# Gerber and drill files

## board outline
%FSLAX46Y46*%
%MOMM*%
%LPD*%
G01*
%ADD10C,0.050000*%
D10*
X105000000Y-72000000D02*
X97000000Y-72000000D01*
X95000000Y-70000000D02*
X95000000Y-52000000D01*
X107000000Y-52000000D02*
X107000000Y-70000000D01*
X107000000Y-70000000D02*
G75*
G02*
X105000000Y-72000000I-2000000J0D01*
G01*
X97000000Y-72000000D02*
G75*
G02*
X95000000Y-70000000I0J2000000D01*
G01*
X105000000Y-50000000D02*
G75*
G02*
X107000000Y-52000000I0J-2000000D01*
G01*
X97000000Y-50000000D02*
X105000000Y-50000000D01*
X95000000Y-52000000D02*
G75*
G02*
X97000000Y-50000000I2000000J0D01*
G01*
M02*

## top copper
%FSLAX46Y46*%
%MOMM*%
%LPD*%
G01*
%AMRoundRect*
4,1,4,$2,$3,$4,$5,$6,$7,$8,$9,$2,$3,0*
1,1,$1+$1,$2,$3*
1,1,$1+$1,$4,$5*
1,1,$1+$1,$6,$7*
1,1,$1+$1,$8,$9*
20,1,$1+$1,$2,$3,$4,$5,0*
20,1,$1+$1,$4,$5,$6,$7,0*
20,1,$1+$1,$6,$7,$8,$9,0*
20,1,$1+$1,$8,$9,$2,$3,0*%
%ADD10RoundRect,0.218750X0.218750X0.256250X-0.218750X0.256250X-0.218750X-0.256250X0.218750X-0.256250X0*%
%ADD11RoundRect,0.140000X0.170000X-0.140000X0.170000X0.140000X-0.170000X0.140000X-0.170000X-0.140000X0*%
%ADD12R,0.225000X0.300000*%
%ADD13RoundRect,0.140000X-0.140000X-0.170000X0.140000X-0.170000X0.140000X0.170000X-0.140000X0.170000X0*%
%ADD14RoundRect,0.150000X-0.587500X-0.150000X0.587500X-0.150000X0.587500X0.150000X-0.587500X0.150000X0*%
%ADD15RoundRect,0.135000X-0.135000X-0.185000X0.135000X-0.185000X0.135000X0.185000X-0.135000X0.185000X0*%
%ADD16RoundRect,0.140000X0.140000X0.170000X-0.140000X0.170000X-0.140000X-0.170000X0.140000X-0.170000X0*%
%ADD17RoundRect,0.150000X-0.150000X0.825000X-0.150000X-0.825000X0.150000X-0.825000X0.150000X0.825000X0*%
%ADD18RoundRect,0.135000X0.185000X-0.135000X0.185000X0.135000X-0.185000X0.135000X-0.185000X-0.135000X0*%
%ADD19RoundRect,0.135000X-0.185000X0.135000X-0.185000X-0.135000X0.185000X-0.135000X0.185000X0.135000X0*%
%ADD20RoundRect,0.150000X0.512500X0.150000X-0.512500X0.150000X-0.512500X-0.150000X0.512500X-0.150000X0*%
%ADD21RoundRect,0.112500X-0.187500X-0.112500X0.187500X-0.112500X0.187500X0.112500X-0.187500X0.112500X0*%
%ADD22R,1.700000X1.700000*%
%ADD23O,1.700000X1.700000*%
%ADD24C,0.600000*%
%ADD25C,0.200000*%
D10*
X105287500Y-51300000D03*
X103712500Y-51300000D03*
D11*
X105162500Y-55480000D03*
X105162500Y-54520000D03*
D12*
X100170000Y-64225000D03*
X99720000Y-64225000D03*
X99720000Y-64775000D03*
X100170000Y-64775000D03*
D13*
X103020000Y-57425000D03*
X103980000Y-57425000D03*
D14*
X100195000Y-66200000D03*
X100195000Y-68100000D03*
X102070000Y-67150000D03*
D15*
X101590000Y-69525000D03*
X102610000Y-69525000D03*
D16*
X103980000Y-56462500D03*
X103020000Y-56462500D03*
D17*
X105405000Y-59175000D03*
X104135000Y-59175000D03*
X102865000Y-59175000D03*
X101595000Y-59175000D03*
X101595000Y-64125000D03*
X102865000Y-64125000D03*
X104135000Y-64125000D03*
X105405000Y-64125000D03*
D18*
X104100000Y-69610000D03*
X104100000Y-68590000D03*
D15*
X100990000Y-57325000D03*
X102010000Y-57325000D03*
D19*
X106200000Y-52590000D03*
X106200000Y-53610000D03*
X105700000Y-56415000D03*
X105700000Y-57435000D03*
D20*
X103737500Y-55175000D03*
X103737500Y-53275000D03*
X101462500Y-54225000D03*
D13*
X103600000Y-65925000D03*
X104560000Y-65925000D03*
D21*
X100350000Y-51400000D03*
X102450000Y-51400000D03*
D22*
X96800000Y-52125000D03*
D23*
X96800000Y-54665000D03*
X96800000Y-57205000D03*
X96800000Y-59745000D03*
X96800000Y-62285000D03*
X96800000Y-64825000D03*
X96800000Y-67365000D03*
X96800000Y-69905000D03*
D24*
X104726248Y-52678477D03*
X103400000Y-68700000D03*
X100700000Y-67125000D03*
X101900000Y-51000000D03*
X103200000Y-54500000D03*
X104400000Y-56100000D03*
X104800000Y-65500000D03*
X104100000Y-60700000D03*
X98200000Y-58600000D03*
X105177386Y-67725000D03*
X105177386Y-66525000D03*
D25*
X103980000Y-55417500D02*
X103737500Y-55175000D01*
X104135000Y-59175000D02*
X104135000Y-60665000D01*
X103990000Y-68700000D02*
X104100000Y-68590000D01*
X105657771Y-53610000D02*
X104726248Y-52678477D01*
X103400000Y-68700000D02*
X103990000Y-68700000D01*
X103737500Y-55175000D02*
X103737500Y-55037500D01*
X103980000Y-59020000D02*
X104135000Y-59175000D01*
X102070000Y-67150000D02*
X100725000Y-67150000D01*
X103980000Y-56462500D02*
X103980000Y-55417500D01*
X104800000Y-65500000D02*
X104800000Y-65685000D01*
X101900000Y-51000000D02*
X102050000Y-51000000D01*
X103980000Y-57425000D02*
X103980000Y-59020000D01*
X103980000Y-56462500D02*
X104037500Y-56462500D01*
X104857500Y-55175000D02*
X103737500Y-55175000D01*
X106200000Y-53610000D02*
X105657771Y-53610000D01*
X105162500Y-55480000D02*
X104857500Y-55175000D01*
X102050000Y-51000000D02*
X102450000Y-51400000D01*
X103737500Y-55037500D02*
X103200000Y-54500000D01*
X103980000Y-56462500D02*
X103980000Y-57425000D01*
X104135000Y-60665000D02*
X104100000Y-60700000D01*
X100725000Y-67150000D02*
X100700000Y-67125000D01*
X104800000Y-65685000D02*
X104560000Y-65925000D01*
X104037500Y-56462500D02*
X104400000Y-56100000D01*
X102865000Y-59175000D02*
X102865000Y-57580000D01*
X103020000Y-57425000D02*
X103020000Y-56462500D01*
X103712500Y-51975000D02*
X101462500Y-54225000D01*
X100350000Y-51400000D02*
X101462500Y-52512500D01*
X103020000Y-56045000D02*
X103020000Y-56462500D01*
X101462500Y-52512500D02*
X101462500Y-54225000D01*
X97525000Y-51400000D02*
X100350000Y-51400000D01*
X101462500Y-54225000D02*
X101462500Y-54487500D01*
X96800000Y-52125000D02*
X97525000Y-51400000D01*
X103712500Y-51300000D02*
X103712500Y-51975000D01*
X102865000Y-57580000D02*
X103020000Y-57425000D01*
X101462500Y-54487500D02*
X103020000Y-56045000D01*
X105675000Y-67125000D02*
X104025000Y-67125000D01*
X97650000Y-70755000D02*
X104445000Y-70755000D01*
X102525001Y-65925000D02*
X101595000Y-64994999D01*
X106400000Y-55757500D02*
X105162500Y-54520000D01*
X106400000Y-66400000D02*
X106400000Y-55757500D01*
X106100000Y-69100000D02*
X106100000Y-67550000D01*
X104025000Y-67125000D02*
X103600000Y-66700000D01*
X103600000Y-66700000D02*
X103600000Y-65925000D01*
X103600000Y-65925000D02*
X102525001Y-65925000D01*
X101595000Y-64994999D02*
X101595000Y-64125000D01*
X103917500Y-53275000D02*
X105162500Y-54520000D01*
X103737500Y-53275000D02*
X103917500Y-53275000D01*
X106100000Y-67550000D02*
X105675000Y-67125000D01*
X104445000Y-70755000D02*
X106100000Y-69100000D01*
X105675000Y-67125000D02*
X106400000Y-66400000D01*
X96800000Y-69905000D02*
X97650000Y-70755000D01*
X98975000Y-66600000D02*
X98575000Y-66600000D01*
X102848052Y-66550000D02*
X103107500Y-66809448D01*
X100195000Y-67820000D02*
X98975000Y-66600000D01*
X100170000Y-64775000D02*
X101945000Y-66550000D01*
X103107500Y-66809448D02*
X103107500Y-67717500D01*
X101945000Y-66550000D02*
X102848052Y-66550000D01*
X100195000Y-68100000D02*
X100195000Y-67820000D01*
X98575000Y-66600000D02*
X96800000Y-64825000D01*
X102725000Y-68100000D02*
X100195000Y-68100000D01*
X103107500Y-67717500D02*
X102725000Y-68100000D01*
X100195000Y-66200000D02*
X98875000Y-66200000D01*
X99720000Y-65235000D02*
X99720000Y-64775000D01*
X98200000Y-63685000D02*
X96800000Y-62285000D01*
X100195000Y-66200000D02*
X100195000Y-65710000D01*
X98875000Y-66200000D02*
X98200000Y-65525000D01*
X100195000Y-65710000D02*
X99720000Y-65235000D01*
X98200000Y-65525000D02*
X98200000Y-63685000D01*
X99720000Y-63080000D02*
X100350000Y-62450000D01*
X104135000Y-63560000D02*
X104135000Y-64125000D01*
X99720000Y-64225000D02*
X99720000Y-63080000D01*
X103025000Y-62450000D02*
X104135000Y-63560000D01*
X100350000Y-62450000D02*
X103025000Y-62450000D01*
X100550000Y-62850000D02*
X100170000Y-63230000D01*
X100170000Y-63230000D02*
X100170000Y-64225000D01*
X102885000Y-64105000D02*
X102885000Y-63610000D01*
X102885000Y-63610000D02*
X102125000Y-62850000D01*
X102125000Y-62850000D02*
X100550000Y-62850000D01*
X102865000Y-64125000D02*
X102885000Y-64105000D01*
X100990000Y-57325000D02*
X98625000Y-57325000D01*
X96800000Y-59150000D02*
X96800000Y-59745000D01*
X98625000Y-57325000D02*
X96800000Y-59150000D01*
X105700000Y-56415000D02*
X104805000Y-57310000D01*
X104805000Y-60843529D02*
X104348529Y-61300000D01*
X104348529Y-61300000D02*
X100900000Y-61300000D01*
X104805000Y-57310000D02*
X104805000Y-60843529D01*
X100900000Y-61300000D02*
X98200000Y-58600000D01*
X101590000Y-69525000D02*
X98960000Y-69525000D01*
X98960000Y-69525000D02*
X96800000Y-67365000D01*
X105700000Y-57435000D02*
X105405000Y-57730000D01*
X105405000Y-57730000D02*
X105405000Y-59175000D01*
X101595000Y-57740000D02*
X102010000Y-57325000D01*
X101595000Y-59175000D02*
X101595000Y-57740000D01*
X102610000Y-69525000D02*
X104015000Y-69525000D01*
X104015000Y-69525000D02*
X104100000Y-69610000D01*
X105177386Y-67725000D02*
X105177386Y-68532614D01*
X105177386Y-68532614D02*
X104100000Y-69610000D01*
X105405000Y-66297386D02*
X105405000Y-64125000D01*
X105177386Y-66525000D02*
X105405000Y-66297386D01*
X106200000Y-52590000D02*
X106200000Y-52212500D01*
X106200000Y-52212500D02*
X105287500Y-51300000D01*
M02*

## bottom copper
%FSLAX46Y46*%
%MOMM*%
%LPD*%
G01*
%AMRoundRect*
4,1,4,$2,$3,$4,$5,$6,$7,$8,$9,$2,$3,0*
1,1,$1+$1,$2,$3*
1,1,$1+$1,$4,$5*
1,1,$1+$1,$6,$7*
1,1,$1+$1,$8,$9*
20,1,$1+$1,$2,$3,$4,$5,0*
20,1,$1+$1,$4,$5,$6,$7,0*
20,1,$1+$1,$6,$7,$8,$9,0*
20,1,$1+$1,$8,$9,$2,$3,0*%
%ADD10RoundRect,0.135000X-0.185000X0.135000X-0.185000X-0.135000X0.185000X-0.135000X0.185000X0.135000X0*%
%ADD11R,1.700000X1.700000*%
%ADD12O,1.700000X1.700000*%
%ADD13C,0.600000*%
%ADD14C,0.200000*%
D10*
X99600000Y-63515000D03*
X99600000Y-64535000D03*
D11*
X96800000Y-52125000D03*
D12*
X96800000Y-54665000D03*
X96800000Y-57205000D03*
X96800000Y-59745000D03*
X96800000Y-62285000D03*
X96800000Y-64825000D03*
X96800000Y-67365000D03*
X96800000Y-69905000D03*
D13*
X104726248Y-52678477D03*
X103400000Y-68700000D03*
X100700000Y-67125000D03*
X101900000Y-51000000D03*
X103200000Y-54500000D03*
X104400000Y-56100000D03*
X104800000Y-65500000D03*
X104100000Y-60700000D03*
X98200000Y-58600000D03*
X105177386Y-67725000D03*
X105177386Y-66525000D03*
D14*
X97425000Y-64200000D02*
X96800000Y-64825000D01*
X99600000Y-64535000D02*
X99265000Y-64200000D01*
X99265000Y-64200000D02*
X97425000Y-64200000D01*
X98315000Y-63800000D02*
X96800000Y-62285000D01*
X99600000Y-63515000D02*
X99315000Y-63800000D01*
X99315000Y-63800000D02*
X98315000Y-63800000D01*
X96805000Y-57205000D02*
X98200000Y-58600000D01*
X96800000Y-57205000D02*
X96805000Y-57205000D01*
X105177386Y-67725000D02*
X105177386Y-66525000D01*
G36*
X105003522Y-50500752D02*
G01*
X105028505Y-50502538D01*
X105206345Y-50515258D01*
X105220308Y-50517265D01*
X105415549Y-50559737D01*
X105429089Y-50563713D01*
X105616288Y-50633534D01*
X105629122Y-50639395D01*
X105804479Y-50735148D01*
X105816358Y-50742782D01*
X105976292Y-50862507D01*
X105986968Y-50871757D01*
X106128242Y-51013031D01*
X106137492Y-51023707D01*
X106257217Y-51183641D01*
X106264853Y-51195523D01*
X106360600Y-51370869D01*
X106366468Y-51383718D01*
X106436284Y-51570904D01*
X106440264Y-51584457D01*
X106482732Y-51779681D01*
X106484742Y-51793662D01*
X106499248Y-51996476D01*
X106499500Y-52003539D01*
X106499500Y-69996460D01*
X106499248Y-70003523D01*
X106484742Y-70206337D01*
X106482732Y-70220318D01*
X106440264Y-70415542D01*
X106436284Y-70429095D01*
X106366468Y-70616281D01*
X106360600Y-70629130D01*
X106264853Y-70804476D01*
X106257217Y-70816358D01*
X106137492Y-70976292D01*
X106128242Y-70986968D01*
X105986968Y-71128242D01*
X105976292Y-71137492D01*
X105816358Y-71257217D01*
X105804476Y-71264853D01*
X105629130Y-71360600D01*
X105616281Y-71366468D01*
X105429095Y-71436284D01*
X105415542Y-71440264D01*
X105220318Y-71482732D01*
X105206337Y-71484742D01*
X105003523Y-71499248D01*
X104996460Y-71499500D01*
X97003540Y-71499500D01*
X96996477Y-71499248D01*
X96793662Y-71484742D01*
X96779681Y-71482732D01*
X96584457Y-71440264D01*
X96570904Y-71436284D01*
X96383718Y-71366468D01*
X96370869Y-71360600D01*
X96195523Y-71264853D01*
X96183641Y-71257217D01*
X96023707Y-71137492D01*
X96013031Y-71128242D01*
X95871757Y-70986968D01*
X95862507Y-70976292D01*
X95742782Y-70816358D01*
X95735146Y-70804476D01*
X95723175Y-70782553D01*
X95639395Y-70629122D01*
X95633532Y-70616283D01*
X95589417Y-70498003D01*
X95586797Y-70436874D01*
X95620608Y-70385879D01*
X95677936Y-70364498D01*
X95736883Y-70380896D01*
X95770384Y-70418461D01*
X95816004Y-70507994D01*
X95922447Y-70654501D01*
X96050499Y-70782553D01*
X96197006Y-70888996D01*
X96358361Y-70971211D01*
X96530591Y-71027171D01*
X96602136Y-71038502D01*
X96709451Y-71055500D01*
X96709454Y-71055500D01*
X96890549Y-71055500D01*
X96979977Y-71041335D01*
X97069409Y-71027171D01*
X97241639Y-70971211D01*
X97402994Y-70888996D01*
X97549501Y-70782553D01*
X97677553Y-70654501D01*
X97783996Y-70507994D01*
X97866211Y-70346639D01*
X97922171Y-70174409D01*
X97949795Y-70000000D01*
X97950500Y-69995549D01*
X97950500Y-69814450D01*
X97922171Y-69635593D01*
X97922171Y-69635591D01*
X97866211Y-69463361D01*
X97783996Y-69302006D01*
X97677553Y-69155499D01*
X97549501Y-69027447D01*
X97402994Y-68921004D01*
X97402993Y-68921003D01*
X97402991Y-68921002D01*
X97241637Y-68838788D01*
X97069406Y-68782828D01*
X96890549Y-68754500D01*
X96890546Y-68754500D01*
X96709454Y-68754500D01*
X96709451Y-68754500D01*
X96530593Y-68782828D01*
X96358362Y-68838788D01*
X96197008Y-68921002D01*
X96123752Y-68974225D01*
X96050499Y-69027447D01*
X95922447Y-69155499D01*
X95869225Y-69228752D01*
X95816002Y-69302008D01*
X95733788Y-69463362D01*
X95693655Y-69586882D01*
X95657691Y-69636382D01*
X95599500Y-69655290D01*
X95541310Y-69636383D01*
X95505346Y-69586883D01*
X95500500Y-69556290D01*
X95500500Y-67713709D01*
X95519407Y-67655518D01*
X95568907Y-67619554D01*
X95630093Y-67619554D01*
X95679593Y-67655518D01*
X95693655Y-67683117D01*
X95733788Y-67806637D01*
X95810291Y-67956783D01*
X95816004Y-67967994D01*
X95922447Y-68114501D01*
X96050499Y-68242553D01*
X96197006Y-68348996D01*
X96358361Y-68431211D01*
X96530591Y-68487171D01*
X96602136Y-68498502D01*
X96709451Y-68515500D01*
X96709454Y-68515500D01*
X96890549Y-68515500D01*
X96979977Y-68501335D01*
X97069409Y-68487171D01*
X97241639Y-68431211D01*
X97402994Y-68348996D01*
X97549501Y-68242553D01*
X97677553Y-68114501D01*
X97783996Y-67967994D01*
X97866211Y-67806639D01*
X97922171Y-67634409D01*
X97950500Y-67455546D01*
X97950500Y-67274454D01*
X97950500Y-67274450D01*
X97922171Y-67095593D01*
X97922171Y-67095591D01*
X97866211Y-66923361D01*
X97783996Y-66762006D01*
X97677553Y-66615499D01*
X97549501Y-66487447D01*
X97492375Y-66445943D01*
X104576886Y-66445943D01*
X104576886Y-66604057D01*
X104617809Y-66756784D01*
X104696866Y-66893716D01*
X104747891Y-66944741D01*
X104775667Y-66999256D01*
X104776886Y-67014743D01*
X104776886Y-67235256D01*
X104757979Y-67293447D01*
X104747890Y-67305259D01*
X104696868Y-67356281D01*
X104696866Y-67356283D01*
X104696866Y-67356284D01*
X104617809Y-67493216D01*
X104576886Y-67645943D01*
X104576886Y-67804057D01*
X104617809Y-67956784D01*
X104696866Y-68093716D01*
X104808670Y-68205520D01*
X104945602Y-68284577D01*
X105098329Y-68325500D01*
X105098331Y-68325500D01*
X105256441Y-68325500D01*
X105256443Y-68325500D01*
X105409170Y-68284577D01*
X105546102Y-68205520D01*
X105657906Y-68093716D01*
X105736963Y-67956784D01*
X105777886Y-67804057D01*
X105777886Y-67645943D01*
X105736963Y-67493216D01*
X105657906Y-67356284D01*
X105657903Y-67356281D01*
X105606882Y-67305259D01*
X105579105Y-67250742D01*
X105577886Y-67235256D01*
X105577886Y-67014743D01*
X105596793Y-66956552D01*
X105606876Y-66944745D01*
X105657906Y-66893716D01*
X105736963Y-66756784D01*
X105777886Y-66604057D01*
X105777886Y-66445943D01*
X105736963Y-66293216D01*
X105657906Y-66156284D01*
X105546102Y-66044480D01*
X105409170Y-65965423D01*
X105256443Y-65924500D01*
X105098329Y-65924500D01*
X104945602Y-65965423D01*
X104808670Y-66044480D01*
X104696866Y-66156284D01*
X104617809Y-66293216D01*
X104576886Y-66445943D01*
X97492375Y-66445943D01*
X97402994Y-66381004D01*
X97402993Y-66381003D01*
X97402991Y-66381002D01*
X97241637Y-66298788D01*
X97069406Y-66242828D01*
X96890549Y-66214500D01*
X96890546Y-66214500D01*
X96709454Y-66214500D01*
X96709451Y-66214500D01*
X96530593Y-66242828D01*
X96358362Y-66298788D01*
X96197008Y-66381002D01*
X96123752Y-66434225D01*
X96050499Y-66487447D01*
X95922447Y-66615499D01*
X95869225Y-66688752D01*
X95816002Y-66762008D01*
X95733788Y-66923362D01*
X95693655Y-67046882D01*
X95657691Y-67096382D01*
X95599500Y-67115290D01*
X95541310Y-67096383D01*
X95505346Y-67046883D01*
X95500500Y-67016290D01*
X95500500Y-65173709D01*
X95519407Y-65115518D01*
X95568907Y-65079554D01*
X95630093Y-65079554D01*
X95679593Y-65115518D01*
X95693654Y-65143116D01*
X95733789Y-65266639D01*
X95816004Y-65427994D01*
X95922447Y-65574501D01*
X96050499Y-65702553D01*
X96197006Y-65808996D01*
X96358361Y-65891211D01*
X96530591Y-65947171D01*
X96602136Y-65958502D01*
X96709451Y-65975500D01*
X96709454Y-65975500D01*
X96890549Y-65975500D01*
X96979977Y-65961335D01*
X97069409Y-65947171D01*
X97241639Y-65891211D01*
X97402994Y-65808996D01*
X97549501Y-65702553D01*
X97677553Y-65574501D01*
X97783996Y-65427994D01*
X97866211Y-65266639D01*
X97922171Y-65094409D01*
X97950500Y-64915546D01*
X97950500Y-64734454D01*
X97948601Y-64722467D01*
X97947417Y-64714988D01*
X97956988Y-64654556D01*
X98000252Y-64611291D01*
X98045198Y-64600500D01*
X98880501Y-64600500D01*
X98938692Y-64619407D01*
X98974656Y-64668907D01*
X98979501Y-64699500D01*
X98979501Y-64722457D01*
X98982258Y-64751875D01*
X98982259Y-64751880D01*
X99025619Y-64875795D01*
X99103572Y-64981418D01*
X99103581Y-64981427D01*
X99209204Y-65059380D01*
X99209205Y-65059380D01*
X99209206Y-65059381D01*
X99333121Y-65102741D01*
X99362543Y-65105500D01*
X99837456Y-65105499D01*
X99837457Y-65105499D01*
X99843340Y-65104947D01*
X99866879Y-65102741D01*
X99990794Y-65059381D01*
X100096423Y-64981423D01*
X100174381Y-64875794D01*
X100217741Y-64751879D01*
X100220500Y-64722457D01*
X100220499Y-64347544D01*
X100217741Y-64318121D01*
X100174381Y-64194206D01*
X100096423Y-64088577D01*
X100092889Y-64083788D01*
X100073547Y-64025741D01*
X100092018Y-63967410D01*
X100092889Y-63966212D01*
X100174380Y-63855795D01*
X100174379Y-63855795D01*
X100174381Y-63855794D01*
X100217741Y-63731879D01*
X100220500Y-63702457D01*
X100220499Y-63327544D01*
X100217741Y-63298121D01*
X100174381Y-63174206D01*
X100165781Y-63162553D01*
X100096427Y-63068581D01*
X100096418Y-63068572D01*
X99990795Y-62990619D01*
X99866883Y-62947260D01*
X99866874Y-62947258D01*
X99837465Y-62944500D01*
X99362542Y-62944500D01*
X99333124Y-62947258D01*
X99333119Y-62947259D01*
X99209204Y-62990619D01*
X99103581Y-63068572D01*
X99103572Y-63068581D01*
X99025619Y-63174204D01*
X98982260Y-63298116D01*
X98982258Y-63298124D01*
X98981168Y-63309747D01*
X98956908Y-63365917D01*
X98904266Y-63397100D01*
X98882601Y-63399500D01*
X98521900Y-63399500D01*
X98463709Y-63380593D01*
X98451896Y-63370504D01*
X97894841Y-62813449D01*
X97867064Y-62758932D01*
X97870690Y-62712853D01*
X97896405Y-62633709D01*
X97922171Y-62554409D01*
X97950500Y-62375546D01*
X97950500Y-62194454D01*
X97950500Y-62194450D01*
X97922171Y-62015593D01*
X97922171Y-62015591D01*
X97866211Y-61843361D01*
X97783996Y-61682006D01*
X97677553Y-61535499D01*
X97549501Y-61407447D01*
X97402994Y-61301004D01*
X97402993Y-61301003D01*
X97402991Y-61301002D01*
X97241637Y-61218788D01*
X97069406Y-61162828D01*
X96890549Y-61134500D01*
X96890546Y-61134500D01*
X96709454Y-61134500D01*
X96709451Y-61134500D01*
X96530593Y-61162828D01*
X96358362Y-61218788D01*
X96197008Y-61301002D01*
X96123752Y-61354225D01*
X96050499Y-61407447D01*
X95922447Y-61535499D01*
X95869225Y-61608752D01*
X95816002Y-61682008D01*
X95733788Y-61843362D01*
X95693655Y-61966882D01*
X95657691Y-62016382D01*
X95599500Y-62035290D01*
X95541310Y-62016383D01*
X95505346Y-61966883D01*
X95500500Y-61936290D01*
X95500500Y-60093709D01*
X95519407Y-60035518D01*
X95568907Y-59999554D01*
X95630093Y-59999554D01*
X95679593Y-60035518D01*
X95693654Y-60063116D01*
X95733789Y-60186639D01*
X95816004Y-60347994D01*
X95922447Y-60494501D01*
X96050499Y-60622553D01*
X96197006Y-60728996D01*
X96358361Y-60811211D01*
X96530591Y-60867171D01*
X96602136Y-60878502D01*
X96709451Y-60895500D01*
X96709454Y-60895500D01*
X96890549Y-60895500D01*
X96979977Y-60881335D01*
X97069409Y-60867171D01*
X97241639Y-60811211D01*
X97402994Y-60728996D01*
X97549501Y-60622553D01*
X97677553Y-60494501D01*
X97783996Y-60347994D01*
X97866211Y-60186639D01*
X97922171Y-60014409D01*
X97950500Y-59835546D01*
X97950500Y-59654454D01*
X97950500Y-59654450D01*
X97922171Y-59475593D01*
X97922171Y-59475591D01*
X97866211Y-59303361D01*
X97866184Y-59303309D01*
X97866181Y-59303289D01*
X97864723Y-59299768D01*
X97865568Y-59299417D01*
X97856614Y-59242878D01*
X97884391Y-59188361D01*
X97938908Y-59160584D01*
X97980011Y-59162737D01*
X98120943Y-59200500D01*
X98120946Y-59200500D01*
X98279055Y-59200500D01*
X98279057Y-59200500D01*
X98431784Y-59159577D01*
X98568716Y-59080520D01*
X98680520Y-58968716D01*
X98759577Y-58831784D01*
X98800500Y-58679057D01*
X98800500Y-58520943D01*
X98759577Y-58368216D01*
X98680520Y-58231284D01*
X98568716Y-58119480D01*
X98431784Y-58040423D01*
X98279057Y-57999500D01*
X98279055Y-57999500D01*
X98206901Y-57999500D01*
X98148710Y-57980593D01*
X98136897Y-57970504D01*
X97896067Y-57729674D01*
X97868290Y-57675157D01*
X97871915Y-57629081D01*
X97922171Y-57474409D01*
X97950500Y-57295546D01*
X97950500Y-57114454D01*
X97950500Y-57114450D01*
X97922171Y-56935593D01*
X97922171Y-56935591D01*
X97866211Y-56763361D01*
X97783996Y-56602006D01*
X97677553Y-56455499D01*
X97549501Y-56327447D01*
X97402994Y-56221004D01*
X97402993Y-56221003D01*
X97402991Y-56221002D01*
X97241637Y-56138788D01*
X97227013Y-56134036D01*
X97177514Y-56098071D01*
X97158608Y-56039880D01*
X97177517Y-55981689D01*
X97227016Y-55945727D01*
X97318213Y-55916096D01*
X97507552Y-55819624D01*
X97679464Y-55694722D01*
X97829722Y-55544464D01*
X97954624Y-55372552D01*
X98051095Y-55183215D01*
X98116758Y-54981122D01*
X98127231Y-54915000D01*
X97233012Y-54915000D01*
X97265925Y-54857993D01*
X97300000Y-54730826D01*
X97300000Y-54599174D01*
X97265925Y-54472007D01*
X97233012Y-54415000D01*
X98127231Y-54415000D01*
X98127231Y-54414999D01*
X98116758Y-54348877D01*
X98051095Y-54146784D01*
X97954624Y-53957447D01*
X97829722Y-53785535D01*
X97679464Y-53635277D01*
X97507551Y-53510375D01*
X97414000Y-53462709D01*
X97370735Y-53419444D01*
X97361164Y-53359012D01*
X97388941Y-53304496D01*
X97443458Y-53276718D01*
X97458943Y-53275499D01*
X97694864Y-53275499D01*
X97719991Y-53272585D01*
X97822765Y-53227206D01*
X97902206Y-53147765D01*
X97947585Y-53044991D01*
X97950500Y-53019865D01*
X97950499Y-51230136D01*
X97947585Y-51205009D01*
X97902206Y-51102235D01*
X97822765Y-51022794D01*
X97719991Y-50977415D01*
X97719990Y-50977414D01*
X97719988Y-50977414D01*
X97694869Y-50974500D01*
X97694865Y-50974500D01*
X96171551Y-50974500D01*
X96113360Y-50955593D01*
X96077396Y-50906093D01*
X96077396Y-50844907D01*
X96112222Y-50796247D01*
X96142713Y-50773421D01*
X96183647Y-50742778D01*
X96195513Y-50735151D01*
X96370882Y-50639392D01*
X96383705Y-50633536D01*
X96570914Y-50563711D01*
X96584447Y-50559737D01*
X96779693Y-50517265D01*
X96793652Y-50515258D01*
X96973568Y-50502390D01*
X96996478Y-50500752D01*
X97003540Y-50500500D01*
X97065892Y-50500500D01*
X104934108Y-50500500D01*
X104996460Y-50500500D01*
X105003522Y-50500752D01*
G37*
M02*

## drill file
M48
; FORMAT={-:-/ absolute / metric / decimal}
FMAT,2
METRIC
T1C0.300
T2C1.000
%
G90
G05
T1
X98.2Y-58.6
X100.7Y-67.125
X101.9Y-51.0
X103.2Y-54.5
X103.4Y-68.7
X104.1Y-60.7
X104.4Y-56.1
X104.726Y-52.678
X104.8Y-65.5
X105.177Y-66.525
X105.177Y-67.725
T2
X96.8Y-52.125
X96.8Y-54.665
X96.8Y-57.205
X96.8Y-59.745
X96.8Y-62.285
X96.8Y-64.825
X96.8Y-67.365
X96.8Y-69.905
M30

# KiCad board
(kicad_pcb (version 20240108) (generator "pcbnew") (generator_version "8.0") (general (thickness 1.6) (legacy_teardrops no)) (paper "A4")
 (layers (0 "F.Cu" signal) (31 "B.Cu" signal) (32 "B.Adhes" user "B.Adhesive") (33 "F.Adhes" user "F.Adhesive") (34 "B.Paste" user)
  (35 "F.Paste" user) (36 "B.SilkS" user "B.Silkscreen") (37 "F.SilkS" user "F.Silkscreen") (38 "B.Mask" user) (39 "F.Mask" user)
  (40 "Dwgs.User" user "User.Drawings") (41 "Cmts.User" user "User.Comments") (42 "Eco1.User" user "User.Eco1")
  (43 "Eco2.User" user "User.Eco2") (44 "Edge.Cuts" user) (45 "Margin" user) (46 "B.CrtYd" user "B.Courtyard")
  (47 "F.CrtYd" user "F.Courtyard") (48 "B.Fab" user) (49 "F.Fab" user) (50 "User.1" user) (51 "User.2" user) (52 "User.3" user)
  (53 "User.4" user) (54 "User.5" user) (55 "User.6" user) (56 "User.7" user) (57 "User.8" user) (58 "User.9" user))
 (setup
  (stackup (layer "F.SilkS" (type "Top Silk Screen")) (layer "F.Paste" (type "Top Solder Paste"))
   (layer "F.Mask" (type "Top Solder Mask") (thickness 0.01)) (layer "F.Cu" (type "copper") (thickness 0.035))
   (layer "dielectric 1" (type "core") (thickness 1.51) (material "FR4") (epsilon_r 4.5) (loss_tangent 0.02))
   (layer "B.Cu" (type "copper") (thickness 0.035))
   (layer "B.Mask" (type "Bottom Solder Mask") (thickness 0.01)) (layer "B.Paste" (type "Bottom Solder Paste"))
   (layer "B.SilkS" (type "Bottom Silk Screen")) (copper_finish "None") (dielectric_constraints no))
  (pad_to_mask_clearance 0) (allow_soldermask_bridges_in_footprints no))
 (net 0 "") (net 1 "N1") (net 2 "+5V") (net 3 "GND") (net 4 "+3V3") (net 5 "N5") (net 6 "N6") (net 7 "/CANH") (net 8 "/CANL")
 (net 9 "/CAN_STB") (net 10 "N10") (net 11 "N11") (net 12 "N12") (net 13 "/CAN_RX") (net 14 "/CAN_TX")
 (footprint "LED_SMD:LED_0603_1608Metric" (layer "F.Cu") (at 104.5 51.3 180)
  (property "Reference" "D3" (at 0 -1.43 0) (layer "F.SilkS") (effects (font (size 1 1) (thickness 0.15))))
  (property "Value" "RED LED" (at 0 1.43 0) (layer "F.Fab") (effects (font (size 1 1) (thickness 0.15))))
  (pad "1" smd roundrect (at -0.7875 0 180) (size 0.875 0.95) (layers "F.Cu" "F.Paste" "F.Mask") (roundrect_rratio 0.25) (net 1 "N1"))
  (pad "2" smd roundrect (at 0.7875 0 180) (size 0.875 0.95) (layers "F.Cu" "F.Paste" "F.Mask") (roundrect_rratio 0.25) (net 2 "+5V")))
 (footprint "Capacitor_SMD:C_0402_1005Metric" (layer "F.Cu") (at 105.1625 55 90)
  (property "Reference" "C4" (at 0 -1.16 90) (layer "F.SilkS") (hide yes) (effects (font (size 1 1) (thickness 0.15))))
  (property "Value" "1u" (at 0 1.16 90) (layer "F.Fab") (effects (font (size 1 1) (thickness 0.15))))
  (pad "1" smd roundrect (at -0.48 0 90) (size 0.56 0.62) (layers "F.Cu" "F.Paste" "F.Mask") (roundrect_rratio 0.25) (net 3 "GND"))
  (pad "2" smd roundrect (at 0.48 0 90) (size 0.56 0.62) (layers "F.Cu" "F.Paste" "F.Mask") (roundrect_rratio 0.25) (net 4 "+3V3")))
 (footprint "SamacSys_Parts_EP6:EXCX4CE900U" (layer "F.Cu") (at 99.945 64.5 180)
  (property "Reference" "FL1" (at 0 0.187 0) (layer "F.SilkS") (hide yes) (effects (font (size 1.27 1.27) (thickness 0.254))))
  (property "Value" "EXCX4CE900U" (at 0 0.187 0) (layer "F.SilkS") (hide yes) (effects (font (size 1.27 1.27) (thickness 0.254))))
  (pad "1" smd rect (at -0.225 0.275 180) (size 0.225 0.3) (layers "F.Cu" "F.Paste" "F.Mask") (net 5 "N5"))
  (pad "2" smd rect (at 0.225 0.275 180) (size 0.225 0.3) (layers "F.Cu" "F.Paste" "F.Mask") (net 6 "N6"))
  (pad "3" smd rect (at 0.225 -0.275 180) (size 0.225 0.3) (layers "F.Cu" "F.Paste" "F.Mask") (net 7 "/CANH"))
  (pad "4" smd rect (at -0.225 -0.275 180) (size 0.225 0.3) (layers "F.Cu" "F.Paste" "F.Mask") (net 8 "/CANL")))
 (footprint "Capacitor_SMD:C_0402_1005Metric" (layer "F.Cu") (at 103.5 57.425)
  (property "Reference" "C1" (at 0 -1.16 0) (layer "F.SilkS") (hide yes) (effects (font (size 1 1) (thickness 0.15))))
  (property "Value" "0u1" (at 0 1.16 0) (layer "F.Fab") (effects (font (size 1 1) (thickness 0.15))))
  (pad "1" smd roundrect (at -0.48 0) (size 0.56 0.62) (layers "F.Cu" "F.Paste" "F.Mask") (roundrect_rratio 0.25) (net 2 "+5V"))
  (pad "2" smd roundrect (at 0.48 0) (size 0.56 0.62) (layers "F.Cu" "F.Paste" "F.Mask") (roundrect_rratio 0.25) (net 3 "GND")))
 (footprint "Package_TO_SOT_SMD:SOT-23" (layer "F.Cu") (at 101.1325 67.15)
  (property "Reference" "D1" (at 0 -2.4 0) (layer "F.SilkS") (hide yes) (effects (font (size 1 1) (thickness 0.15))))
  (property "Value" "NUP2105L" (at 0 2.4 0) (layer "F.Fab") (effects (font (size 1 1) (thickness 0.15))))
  (pad "1" smd roundrect (at -0.9375 -0.95) (size 1.475 0.6) (layers "F.Cu" "F.Paste" "F.Mask") (roundrect_rratio 0.25) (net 7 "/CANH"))
  (pad "2" smd roundrect (at -0.9375 0.95) (size 1.475 0.6) (layers "F.Cu" "F.Paste" "F.Mask") (roundrect_rratio 0.25) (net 8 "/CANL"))
  (pad "3" smd roundrect (at 0.9375 0) (size 1.475 0.6) (layers "F.Cu" "F.Paste" "F.Mask") (roundrect_rratio 0.25) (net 3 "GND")))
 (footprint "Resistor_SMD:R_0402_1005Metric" (layer "F.Cu") (at 102.1 69.525)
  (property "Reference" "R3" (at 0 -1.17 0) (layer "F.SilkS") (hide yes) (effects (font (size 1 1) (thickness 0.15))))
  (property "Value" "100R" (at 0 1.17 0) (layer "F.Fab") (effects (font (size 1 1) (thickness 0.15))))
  (pad "1" smd roundrect (at -0.51 0) (size 0.54 0.64) (layers "F.Cu" "F.Paste" "F.Mask") (roundrect_rratio 0.25) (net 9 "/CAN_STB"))
  (pad "2" smd roundrect (at 0.51 0) (size 0.54 0.64) (layers "F.Cu" "F.Paste" "F.Mask") (roundrect_rratio 0.25) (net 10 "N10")))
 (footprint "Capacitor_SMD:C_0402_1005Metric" (layer "F.Cu") (at 103.5 56.4625 180)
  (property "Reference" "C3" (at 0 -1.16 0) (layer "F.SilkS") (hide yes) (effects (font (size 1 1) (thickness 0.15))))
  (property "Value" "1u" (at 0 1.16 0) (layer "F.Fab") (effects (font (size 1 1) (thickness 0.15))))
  (pad "1" smd roundrect (at -0.48 0 180) (size 0.56 0.62) (layers "F.Cu" "F.Paste" "F.Mask") (roundrect_rratio 0.25) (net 3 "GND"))
  (pad "2" smd roundrect (at 0.48 0 180) (size 0.56 0.62) (layers "F.Cu" "F.Paste" "F.Mask") (roundrect_rratio 0.25) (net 2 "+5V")))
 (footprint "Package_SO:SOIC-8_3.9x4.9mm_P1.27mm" (layer "F.Cu") (at 103.5 61.65 -90)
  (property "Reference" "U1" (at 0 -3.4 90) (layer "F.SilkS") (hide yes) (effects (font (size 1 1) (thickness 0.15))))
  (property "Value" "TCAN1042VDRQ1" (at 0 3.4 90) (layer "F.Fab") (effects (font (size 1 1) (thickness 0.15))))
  (pad "1" smd roundrect (at -2.475 -1.905 270) (size 1.95 0.6) (layers "F.Cu" "F.Paste" "F.Mask") (roundrect_rratio 0.25) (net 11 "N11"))
  (pad "2" smd roundrect (at -2.475 -0.635 270) (size 1.95 0.6) (layers "F.Cu" "F.Paste" "F.Mask") (roundrect_rratio 0.25) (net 3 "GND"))
  (pad "3" smd roundrect (at -2.475 0.635 270) (size 1.95 0.6) (layers "F.Cu" "F.Paste" "F.Mask") (roundrect_rratio 0.25) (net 2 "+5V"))
  (pad "4" smd roundrect (at -2.475 1.905 270) (size 1.95 0.6) (layers "F.Cu" "F.Paste" "F.Mask") (roundrect_rratio 0.25) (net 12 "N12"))
  (pad "5" smd roundrect (at 2.475 1.905 270) (size 1.95 0.6) (layers "F.Cu" "F.Paste" "F.Mask") (roundrect_rratio 0.25) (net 4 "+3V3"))
  (pad "6" smd roundrect (at 2.475 0.635 270) (size 1.95 0.6) (layers "F.Cu" "F.Paste" "F.Mask") (roundrect_rratio 0.25) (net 5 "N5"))
  (pad "7" smd roundrect (at 2.475 -0.635 270) (size 1.95 0.6) (layers "F.Cu" "F.Paste" "F.Mask") (roundrect_rratio 0.25) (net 6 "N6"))
  (pad "8" smd roundrect (at 2.475 -1.905 270) (size 1.95 0.6) (layers "F.Cu" "F.Paste" "F.Mask") (roundrect_rratio 0.25) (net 10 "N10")))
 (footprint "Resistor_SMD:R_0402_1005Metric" (layer "F.Cu") (at 104.1 69.1 90)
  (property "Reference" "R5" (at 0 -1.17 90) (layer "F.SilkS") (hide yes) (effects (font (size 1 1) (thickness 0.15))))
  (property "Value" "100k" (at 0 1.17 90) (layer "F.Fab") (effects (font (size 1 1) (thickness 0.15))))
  (pad "1" smd roundrect (at -0.51 0 90) (size 0.54 0.64) (layers "F.Cu" "F.Paste" "F.Mask") (roundrect_rratio 0.25) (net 10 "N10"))
  (pad "2" smd roundrect (at 0.51 0 90) (size 0.54 0.64) (layers "F.Cu" "F.Paste" "F.Mask") (roundrect_rratio 0.25) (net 3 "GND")))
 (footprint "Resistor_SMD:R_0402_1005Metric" (layer "F.Cu") (at 101.5 57.325)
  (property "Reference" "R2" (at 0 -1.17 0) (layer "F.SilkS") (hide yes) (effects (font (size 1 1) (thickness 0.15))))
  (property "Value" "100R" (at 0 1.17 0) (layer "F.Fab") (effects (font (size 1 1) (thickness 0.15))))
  (pad "1" smd roundrect (at -0.51 0) (size 0.54 0.64) (layers "F.Cu" "F.Paste" "F.Mask") (roundrect_rratio 0.25) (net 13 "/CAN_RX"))
  (pad "2" smd roundrect (at 0.51 0) (size 0.54 0.64) (layers "F.Cu" "F.Paste" "F.Mask") (roundrect_rratio 0.25) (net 12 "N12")))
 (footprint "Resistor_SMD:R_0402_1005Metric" (layer "F.Cu") (at 106.2 53.1 -90)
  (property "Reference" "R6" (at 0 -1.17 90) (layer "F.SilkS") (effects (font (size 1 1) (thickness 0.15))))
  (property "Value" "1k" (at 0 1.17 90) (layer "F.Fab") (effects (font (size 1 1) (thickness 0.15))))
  (pad "1" smd roundrect (at -0.51 0 270) (size 0.54 0.64) (layers "F.Cu" "F.Paste" "F.Mask") (roundrect_rratio 0.25) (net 1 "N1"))
  (pad "2" smd roundrect (at 0.51 0 270) (size 0.54 0.64) (layers "F.Cu" "F.Paste" "F.Mask") (roundrect_rratio 0.25) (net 3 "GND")))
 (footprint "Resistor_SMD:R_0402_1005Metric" (layer "F.Cu") (at 105.7 56.925 -90)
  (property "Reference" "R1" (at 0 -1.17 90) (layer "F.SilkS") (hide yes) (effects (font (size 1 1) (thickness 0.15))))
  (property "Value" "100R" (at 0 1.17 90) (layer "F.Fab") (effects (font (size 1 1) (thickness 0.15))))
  (pad "1" smd roundrect (at -0.51 0 270) (size 0.54 0.64) (layers "F.Cu" "F.Paste" "F.Mask") (roundrect_rratio 0.25) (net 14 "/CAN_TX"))
  (pad "2" smd roundrect (at 0.51 0 270) (size 0.54 0.64) (layers "F.Cu" "F.Paste" "F.Mask") (roundrect_rratio 0.25) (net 11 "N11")))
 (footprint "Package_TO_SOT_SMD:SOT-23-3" (layer "F.Cu") (at 102.6 54.225 180)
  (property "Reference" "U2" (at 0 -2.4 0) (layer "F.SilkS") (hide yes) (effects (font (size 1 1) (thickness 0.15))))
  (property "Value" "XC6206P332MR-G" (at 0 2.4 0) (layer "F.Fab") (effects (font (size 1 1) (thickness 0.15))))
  (pad "1" smd roundrect (at -1.1375 -0.95 180) (size 1.325 0.6) (layers "F.Cu" "F.Paste" "F.Mask") (roundrect_rratio 0.25) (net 3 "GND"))
  (pad "2" smd roundrect (at -1.1375 0.95 180) (size 1.325 0.6) (layers "F.Cu" "F.Paste" "F.Mask") (roundrect_rratio 0.25) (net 4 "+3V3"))
  (pad "3" smd roundrect (at 1.1375 0 180) (size 1.325 0.6) (layers "F.Cu" "F.Paste" "F.Mask") (roundrect_rratio 0.25) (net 2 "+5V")))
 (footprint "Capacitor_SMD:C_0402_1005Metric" (layer "F.Cu") (at 104.08 65.925)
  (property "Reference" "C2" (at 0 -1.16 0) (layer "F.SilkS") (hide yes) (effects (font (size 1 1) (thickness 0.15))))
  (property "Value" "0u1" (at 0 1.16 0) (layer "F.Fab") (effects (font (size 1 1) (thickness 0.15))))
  (pad "1" smd roundrect (at -0.48 0) (size 0.56 0.62) (layers "F.Cu" "F.Paste" "F.Mask") (roundrect_rratio 0.25) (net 4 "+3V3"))
  (pad "2" smd roundrect (at 0.48 0) (size 0.56 0.62) (layers "F.Cu" "F.Paste" "F.Mask") (roundrect_rratio 0.25) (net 3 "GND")))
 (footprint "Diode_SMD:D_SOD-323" (layer "F.Cu") (at 101.4 51.4)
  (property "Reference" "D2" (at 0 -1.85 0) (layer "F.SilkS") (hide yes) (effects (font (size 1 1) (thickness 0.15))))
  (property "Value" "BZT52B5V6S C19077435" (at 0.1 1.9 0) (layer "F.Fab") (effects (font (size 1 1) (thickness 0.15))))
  (pad "1" smd roundrect (at -1.05 0) (size 0.6 0.45) (layers "F.Cu" "F.Paste" "F.Mask") (roundrect_rratio 0.25) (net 2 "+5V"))
  (pad "2" smd roundrect (at 1.05 0) (size 0.6 0.45) (layers "F.Cu" "F.Paste" "F.Mask") (roundrect_rratio 0.25) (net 3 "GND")))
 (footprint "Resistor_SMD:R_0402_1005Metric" (layer "B.Cu") (at 99.6 64.025 -90)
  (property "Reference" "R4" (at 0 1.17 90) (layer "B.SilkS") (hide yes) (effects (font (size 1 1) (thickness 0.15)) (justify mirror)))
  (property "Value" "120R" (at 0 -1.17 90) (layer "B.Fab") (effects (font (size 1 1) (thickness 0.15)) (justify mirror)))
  (pad "1" smd roundrect (at -0.51 0 270) (size 0.54 0.64) (layers "B.Cu" "B.Paste" "B.Mask") (roundrect_rratio 0.25) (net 7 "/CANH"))
  (pad "2" smd roundrect (at 0.51 0 270) (size 0.54 0.64) (layers "B.Cu" "B.Paste" "B.Mask") (roundrect_rratio 0.25) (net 8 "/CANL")))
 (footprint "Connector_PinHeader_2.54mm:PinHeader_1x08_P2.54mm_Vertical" (layer "B.Cu") (at 96.8 52.125 180)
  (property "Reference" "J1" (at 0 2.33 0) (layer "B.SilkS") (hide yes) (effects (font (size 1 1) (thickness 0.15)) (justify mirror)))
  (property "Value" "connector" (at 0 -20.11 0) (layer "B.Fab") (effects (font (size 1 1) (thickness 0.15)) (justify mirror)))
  (pad "1" thru_hole rect (at 0 0 180) (size 1.7 1.7) (drill 1) (layers "*.Cu" "*.Mask") (remove_unused_layers no) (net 2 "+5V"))
  (pad "2" thru_hole oval (at 0 -2.54 180) (size 1.7 1.7) (drill 1) (layers "*.Cu" "*.Mask") (remove_unused_layers no) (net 3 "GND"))
  (pad "3" thru_hole oval (at 0 -5.08 180) (size 1.7 1.7) (drill 1) (layers "*.Cu" "*.Mask") (remove_unused_layers no) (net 14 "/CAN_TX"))
  (pad "4" thru_hole oval (at 0 -7.62 180) (size 1.7 1.7) (drill 1) (layers "*.Cu" "*.Mask") (remove_unused_layers no) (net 13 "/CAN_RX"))
  (pad "5" thru_hole oval (at 0 -10.16 180) (size 1.7 1.7) (drill 1) (layers "*.Cu" "*.Mask") (remove_unused_layers no) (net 7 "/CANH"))
  (pad "6" thru_hole oval (at 0 -12.7 180) (size 1.7 1.7) (drill 1) (layers "*.Cu" "*.Mask") (remove_unused_layers no) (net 8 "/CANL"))
  (pad "7" thru_hole oval (at 0 -15.24 180) (size 1.7 1.7) (drill 1) (layers "*.Cu" "*.Mask") (remove_unused_layers no) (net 9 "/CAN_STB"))
  (pad "8" thru_hole oval (at 0 -17.78 180) (size 1.7 1.7) (drill 1) (layers "*.Cu" "*.Mask") (remove_unused_layers no) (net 4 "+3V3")))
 (gr_line (start 105 72) (end 97 72) (stroke (width 0.05) (type default)) (layer "Edge.Cuts"))
 (gr_line (start 95 70) (end 95 52) (stroke (width 0.05) (type default)) (layer "Edge.Cuts"))
 (gr_line (start 107 52) (end 107 70) (stroke (width 0.05) (type default)) (layer "Edge.Cuts"))
 (gr_arc (start 107 70) (mid 106.414214 71.414214) (end 105 72) (stroke (width 0.05) (type default)) (layer "Edge.Cuts"))
 (gr_arc (start 97 72) (mid 95.585786 71.414214) (end 95 70) (stroke (width 0.05) (type default)) (layer "Edge.Cuts"))
 (gr_arc (start 105 50) (mid 106.414214 50.585786) (end 107 52) (stroke (width 0.05) (type default)) (layer "Edge.Cuts"))
 (gr_line (start 97 50) (end 105 50) (stroke (width 0.05) (type default)) (layer "Edge.Cuts"))
 (gr_arc (start 95 52) (mid 95.585786 50.585786) (end 97 50) (stroke (width 0.05) (type default)) (layer "Edge.Cuts"))
 (segment (start 103.98 55.4175) (end 103.7375 55.175) (width 0.2) (layer "F.Cu") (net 3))
 (segment (start 104.135 59.175) (end 104.135 60.665) (width 0.2) (layer "F.Cu") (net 3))
 (segment (start 103.99 68.7) (end 104.1 68.59) (width 0.2) (layer "F.Cu") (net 3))
 (segment (start 105.657771 53.61) (end 104.726248 52.678477) (width 0.2) (layer "F.Cu") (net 3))
 (segment (start 103.4 68.7) (end 103.99 68.7) (width 0.2) (layer "F.Cu") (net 3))
 (segment (start 103.7375 55.175) (end 103.7375 55.0375) (width 0.2) (layer "F.Cu") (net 3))
 (segment (start 103.98 59.02) (end 104.135 59.175) (width 0.2) (layer "F.Cu") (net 3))
 (segment (start 102.07 67.15) (end 100.725 67.15) (width 0.2) (layer "F.Cu") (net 3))
 (segment (start 103.98 56.4625) (end 103.98 55.4175) (width 0.2) (layer "F.Cu") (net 3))
 (segment (start 104.8 65.5) (end 104.8 65.685) (width 0.2) (layer "F.Cu") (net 3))
 (segment (start 101.9 51) (end 102.05 51) (width 0.2) (layer "F.Cu") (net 3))
 (segment (start 103.98 57.425) (end 103.98 59.02) (width 0.2) (layer "F.Cu") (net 3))
 (segment (start 103.98 56.4625) (end 104.0375 56.4625) (width 0.2) (layer "F.Cu") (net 3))
 (segment (start 104.8575 55.175) (end 103.7375 55.175) (width 0.2) (layer "F.Cu") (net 3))
 (segment (start 106.2 53.61) (end 105.657771 53.61) (width 0.2) (layer "F.Cu") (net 3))
 (segment (start 105.1625 55.48) (end 104.8575 55.175) (width 0.2) (layer "F.Cu") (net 3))
 (segment (start 102.05 51) (end 102.45 51.4) (width 0.2) (layer "F.Cu") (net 3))
 (segment (start 103.7375 55.0375) (end 103.2 54.5) (width 0.2) (layer "F.Cu") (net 3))
 (segment (start 103.98 56.4625) (end 103.98 57.425) (width 0.2) (layer "F.Cu") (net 3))
 (segment (start 104.135 60.665) (end 104.1 60.7) (width 0.2) (layer "F.Cu") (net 3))
 (segment (start 100.725 67.15) (end 100.7 67.125) (width 0.2) (layer "F.Cu") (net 3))
 (segment (start 104.8 65.685) (end 104.56 65.925) (width 0.2) (layer "F.Cu") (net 3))
 (segment (start 104.0375 56.4625) (end 104.4 56.1) (width 0.2) (layer "F.Cu") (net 3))
 (via (at 104.726248 52.678477) (size 0.6) (drill 0.3) (layers "F.Cu" "B.Cu") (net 3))
 (via (at 103.4 68.7) (size 0.6) (drill 0.3) (layers "F.Cu" "B.Cu") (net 3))
 (via (at 100.7 67.125) (size 0.6) (drill 0.3) (layers "F.Cu" "B.Cu") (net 3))
 (via (at 101.9 51) (size 0.6) (drill 0.3) (layers "F.Cu" "B.Cu") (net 3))
 (via (at 103.2 54.5) (size 0.6) (drill 0.3) (layers "F.Cu" "B.Cu") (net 3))
 (via (at 104.4 56.1) (size 0.6) (drill 0.3) (layers "F.Cu" "B.Cu") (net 3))
 (via (at 104.8 65.5) (size 0.6) (drill 0.3) (layers "F.Cu" "B.Cu") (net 3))
 (via (at 104.1 60.7) (size 0.6) (drill 0.3) (layers "F.Cu" "B.Cu") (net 3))
 (segment (start 102.865 59.175) (end 102.865 57.58) (width 0.2) (layer "F.Cu") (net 2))
 (segment (start 103.02 57.425) (end 103.02 56.4625) (width 0.2) (layer "F.Cu") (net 2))
 (segment (start 103.7125 51.975) (end 101.4625 54.225) (width 0.2) (layer "F.Cu") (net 2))
 (segment (start 100.35 51.4) (end 101.4625 52.5125) (width 0.2) (layer "F.Cu") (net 2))
 (segment (start 103.02 56.045) (end 103.02 56.4625) (width 0.2) (layer "F.Cu") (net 2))
 (segment (start 101.4625 52.5125) (end 101.4625 54.225) (width 0.2) (layer "F.Cu") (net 2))
 (segment (start 97.525 51.4) (end 100.35 51.4) (width 0.2) (layer "F.Cu") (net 2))
 (segment (start 101.4625 54.225) (end 101.4625 54.4875) (width 0.2) (layer "F.Cu") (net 2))
 (segment (start 96.8 52.125) (end 97.525 51.4) (width 0.2) (layer "F.Cu") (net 2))
 (segment (start 103.7125 51.3) (end 103.7125 51.975) (width 0.2) (layer "F.Cu") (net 2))
 (segment (start 102.865 57.58) (end 103.02 57.425) (width 0.2) (layer "F.Cu") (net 2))
 (segment (start 101.4625 54.4875) (end 103.02 56.045) (width 0.2) (layer "F.Cu") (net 2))
 (segment (start 105.675 67.125) (end 104.025 67.125) (width 0.2) (layer "F.Cu") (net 4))
 (segment (start 97.65 70.755) (end 104.445 70.755) (width 0.2) (layer "F.Cu") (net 4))
 (segment (start 102.525001 65.925) (end 101.595 64.994999) (width 0.2) (layer "F.Cu") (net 4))
 (segment (start 106.4 55.7575) (end 105.1625 54.52) (width 0.2) (layer "F.Cu") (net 4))
 (segment (start 106.4 66.4) (end 106.4 55.7575) (width 0.2) (layer "F.Cu") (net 4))
 (segment (start 106.1 69.1) (end 106.1 67.55) (width 0.2) (layer "F.Cu") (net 4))
 (segment (start 104.025 67.125) (end 103.6 66.7) (width 0.2) (layer "F.Cu") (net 4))
 (segment (start 103.6 66.7) (end 103.6 65.925) (width 0.2) (layer "F.Cu") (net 4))
 (segment (start 103.6 65.925) (end 102.525001 65.925) (width 0.2) (layer "F.Cu") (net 4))
 (segment (start 101.595 64.994999) (end 101.595 64.125) (width 0.2) (layer "F.Cu") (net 4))
 (segment (start 103.9175 53.275) (end 105.1625 54.52) (width 0.2) (layer "F.Cu") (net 4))
 (segment (start 103.7375 53.275) (end 103.9175 53.275) (width 0.2) (layer "F.Cu") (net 4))
 (segment (start 106.1 67.55) (end 105.675 67.125) (width 0.2) (layer "F.Cu") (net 4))
 (segment (start 104.445 70.755) (end 106.1 69.1) (width 0.2) (layer "F.Cu") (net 4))
 (segment (start 105.675 67.125) (end 106.4 66.4) (width 0.2) (layer "F.Cu") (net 4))
 (segment (start 96.8 69.905) (end 97.65 70.755) (width 0.2) (layer "F.Cu") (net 4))
 (segment (start 98.975 66.6) (end 98.575 66.6) (width 0.2) (layer "F.Cu") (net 8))
 (segment (start 102.848052 66.55) (end 103.1075 66.809448) (width 0.2) (layer "F.Cu") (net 8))
 (segment (start 100.195 67.82) (end 98.975 66.6) (width 0.2) (layer "F.Cu") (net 8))
 (segment (start 100.17 64.775) (end 101.945 66.55) (width 0.2) (layer "F.Cu") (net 8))
 (segment (start 103.1075 66.809448) (end 103.1075 67.7175) (width 0.2) (layer "F.Cu") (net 8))
 (segment (start 101.945 66.55) (end 102.848052 66.55) (width 0.2) (layer "F.Cu") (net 8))
 (segment (start 100.195 68.1) (end 100.195 67.82) (width 0.2) (layer "F.Cu") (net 8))
 (segment (start 98.575 66.6) (end 96.8 64.825) (width 0.2) (layer "F.Cu") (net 8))
 (segment (start 102.725 68.1) (end 100.195 68.1) (width 0.2) (layer "F.Cu") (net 8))
 (segment (start 103.1075 67.7175) (end 102.725 68.1) (width 0.2) (layer "F.Cu") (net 8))
 (segment (start 97.425 64.2) (end 96.8 64.825) (width 0.2) (layer "B.Cu") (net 8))
 (segment (start 99.6 64.535) (end 99.265 64.2) (width 0.2) (layer "B.Cu") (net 8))
 (segment (start 99.265 64.2) (end 97.425 64.2) (width 0.2) (layer "B.Cu") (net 8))
 (segment (start 100.195 66.2) (end 98.875 66.2) (width 0.2) (layer "F.Cu") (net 7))
 (segment (start 99.72 65.235) (end 99.72 64.775) (width 0.2) (layer "F.Cu") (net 7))
 (segment (start 98.2 63.685) (end 96.8 62.285) (width 0.2) (layer "F.Cu") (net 7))
 (segment (start 100.195 66.2) (end 100.195 65.71) (width 0.2) (layer "F.Cu") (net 7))
 (segment (start 98.875 66.2) (end 98.2 65.525) (width 0.2) (layer "F.Cu") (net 7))
 (segment (start 100.195 65.71) (end 99.72 65.235) (width 0.2) (layer "F.Cu") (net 7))
 (segment (start 98.2 65.525) (end 98.2 63.685) (width 0.2) (layer "F.Cu") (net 7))
 (segment (start 98.315 63.8) (end 96.8 62.285) (width 0.2) (layer "B.Cu") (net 7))
 (segment (start 99.6 63.515) (end 99.315 63.8) (width 0.2) (layer "B.Cu") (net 7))
 (segment (start 99.315 63.8) (end 98.315 63.8) (width 0.2) (layer "B.Cu") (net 7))
 (segment (start 99.72 63.08) (end 100.35 62.45) (width 0.2) (layer "F.Cu") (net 6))
 (segment (start 104.135 63.56) (end 104.135 64.125) (width 0.2) (layer "F.Cu") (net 6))
 (segment (start 99.72 64.225) (end 99.72 63.08) (width 0.2) (layer "F.Cu") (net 6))
 (segment (start 103.025 62.45) (end 104.135 63.56) (width 0.2) (layer "F.Cu") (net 6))
 (segment (start 100.35 62.45) (end 103.025 62.45) (width 0.2) (layer "F.Cu") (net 6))
 (segment (start 100.55 62.85) (end 100.17 63.23) (width 0.2) (layer "F.Cu") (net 5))
 (segment (start 100.17 63.23) (end 100.17 64.225) (width 0.2) (layer "F.Cu") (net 5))
 (segment (start 102.885 64.105) (end 102.885 63.61) (width 0.2) (layer "F.Cu") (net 5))
 (segment (start 102.885 63.61) (end 102.125 62.85) (width 0.2) (layer "F.Cu") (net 5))
 (segment (start 102.125 62.85) (end 100.55 62.85) (width 0.2) (layer "F.Cu") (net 5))
 (segment (start 102.865 64.125) (end 102.885 64.105) (width 0.2) (layer "F.Cu") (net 5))
 (segment (start 100.99 57.325) (end 98.625 57.325) (width 0.2) (layer "F.Cu") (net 13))
 (segment (start 96.8 59.15) (end 96.8 59.745) (width 0.2) (layer "F.Cu") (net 13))
 (segment (start 98.625 57.325) (end 96.8 59.15) (width 0.2) (layer "F.Cu") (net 13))
 (segment (start 105.7 56.415) (end 104.805 57.31) (width 0.2) (layer "F.Cu") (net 14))
 (segment (start 104.805 60.843529) (end 104.348529 61.3) (width 0.2) (layer "F.Cu") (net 14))
 (segment (start 104.348529 61.3) (end 100.9 61.3) (width 0.2) (layer "F.Cu") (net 14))
 (segment (start 104.805 57.31) (end 104.805 60.843529) (width 0.2) (layer "F.Cu") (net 14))
 (segment (start 100.9 61.3) (end 98.2 58.6) (width 0.2) (layer "F.Cu") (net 14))
 (via (at 98.2 58.6) (size 0.6) (drill 0.3) (layers "F.Cu" "B.Cu") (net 14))
 (segment (start 96.805 57.205) (end 98.2 58.6) (width 0.2) (layer "B.Cu") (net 14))
 (segment (start 96.8 57.205) (end 96.805 57.205) (width 0.2) (layer "B.Cu") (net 14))
 (segment (start 101.59 69.525) (end 98.96 69.525) (width 0.2) (layer "F.Cu") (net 9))
 (segment (start 98.96 69.525) (end 96.8 67.365) (width 0.2) (layer "F.Cu") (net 9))
 (segment (start 105.7 57.435) (end 105.405 57.73) (width 0.2) (layer "F.Cu") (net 11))
 (segment (start 105.405 57.73) (end 105.405 59.175) (width 0.2) (layer "F.Cu") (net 11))
 (segment (start 101.595 57.74) (end 102.01 57.325) (width 0.2) (layer "F.Cu") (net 12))
 (segment (start 101.595 59.175) (end 101.595 57.74) (width 0.2) (layer "F.Cu") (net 12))
 (segment (start 102.61 69.525) (end 104.015 69.525) (width 0.2) (layer "F.Cu") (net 10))
 (segment (start 104.015 69.525) (end 104.1 69.61) (width 0.2) (layer "F.Cu") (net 10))
 (segment (start 105.177386 67.725) (end 105.177386 68.532614) (width 0.2) (layer "F.Cu") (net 10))
 (segment (start 105.177386 68.532614) (end 104.1 69.61) (width 0.2) (layer "F.Cu") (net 10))
 (segment (start 105.405 66.297386) (end 105.405 64.125) (width 0.2) (layer "F.Cu") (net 10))
 (segment (start 105.177386 66.525) (end 105.405 66.297386) (width 0.2) (layer "F.Cu") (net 10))
 (via (at 105.177386 67.725) (size 0.6) (drill 0.3) (layers "F.Cu" "B.Cu") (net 10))
 (via (at 105.177386 66.525) (size 0.6) (drill 0.3) (layers "F.Cu" "B.Cu") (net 10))
 (segment (start 105.177386 67.725) (end 105.177386 66.525) (width 0.2) (layer "B.Cu") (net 10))
 (segment (start 106.2 52.59) (end 106.2 52.2125) (width 0.2) (layer "F.Cu") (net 1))
 (segment (start 106.2 52.2125) (end 105.2875 51.3) (width 0.2) (layer "F.Cu") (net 1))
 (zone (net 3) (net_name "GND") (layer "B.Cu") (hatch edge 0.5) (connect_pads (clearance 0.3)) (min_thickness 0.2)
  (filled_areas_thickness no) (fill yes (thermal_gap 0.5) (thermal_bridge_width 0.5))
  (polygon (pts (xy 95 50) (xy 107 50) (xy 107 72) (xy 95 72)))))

